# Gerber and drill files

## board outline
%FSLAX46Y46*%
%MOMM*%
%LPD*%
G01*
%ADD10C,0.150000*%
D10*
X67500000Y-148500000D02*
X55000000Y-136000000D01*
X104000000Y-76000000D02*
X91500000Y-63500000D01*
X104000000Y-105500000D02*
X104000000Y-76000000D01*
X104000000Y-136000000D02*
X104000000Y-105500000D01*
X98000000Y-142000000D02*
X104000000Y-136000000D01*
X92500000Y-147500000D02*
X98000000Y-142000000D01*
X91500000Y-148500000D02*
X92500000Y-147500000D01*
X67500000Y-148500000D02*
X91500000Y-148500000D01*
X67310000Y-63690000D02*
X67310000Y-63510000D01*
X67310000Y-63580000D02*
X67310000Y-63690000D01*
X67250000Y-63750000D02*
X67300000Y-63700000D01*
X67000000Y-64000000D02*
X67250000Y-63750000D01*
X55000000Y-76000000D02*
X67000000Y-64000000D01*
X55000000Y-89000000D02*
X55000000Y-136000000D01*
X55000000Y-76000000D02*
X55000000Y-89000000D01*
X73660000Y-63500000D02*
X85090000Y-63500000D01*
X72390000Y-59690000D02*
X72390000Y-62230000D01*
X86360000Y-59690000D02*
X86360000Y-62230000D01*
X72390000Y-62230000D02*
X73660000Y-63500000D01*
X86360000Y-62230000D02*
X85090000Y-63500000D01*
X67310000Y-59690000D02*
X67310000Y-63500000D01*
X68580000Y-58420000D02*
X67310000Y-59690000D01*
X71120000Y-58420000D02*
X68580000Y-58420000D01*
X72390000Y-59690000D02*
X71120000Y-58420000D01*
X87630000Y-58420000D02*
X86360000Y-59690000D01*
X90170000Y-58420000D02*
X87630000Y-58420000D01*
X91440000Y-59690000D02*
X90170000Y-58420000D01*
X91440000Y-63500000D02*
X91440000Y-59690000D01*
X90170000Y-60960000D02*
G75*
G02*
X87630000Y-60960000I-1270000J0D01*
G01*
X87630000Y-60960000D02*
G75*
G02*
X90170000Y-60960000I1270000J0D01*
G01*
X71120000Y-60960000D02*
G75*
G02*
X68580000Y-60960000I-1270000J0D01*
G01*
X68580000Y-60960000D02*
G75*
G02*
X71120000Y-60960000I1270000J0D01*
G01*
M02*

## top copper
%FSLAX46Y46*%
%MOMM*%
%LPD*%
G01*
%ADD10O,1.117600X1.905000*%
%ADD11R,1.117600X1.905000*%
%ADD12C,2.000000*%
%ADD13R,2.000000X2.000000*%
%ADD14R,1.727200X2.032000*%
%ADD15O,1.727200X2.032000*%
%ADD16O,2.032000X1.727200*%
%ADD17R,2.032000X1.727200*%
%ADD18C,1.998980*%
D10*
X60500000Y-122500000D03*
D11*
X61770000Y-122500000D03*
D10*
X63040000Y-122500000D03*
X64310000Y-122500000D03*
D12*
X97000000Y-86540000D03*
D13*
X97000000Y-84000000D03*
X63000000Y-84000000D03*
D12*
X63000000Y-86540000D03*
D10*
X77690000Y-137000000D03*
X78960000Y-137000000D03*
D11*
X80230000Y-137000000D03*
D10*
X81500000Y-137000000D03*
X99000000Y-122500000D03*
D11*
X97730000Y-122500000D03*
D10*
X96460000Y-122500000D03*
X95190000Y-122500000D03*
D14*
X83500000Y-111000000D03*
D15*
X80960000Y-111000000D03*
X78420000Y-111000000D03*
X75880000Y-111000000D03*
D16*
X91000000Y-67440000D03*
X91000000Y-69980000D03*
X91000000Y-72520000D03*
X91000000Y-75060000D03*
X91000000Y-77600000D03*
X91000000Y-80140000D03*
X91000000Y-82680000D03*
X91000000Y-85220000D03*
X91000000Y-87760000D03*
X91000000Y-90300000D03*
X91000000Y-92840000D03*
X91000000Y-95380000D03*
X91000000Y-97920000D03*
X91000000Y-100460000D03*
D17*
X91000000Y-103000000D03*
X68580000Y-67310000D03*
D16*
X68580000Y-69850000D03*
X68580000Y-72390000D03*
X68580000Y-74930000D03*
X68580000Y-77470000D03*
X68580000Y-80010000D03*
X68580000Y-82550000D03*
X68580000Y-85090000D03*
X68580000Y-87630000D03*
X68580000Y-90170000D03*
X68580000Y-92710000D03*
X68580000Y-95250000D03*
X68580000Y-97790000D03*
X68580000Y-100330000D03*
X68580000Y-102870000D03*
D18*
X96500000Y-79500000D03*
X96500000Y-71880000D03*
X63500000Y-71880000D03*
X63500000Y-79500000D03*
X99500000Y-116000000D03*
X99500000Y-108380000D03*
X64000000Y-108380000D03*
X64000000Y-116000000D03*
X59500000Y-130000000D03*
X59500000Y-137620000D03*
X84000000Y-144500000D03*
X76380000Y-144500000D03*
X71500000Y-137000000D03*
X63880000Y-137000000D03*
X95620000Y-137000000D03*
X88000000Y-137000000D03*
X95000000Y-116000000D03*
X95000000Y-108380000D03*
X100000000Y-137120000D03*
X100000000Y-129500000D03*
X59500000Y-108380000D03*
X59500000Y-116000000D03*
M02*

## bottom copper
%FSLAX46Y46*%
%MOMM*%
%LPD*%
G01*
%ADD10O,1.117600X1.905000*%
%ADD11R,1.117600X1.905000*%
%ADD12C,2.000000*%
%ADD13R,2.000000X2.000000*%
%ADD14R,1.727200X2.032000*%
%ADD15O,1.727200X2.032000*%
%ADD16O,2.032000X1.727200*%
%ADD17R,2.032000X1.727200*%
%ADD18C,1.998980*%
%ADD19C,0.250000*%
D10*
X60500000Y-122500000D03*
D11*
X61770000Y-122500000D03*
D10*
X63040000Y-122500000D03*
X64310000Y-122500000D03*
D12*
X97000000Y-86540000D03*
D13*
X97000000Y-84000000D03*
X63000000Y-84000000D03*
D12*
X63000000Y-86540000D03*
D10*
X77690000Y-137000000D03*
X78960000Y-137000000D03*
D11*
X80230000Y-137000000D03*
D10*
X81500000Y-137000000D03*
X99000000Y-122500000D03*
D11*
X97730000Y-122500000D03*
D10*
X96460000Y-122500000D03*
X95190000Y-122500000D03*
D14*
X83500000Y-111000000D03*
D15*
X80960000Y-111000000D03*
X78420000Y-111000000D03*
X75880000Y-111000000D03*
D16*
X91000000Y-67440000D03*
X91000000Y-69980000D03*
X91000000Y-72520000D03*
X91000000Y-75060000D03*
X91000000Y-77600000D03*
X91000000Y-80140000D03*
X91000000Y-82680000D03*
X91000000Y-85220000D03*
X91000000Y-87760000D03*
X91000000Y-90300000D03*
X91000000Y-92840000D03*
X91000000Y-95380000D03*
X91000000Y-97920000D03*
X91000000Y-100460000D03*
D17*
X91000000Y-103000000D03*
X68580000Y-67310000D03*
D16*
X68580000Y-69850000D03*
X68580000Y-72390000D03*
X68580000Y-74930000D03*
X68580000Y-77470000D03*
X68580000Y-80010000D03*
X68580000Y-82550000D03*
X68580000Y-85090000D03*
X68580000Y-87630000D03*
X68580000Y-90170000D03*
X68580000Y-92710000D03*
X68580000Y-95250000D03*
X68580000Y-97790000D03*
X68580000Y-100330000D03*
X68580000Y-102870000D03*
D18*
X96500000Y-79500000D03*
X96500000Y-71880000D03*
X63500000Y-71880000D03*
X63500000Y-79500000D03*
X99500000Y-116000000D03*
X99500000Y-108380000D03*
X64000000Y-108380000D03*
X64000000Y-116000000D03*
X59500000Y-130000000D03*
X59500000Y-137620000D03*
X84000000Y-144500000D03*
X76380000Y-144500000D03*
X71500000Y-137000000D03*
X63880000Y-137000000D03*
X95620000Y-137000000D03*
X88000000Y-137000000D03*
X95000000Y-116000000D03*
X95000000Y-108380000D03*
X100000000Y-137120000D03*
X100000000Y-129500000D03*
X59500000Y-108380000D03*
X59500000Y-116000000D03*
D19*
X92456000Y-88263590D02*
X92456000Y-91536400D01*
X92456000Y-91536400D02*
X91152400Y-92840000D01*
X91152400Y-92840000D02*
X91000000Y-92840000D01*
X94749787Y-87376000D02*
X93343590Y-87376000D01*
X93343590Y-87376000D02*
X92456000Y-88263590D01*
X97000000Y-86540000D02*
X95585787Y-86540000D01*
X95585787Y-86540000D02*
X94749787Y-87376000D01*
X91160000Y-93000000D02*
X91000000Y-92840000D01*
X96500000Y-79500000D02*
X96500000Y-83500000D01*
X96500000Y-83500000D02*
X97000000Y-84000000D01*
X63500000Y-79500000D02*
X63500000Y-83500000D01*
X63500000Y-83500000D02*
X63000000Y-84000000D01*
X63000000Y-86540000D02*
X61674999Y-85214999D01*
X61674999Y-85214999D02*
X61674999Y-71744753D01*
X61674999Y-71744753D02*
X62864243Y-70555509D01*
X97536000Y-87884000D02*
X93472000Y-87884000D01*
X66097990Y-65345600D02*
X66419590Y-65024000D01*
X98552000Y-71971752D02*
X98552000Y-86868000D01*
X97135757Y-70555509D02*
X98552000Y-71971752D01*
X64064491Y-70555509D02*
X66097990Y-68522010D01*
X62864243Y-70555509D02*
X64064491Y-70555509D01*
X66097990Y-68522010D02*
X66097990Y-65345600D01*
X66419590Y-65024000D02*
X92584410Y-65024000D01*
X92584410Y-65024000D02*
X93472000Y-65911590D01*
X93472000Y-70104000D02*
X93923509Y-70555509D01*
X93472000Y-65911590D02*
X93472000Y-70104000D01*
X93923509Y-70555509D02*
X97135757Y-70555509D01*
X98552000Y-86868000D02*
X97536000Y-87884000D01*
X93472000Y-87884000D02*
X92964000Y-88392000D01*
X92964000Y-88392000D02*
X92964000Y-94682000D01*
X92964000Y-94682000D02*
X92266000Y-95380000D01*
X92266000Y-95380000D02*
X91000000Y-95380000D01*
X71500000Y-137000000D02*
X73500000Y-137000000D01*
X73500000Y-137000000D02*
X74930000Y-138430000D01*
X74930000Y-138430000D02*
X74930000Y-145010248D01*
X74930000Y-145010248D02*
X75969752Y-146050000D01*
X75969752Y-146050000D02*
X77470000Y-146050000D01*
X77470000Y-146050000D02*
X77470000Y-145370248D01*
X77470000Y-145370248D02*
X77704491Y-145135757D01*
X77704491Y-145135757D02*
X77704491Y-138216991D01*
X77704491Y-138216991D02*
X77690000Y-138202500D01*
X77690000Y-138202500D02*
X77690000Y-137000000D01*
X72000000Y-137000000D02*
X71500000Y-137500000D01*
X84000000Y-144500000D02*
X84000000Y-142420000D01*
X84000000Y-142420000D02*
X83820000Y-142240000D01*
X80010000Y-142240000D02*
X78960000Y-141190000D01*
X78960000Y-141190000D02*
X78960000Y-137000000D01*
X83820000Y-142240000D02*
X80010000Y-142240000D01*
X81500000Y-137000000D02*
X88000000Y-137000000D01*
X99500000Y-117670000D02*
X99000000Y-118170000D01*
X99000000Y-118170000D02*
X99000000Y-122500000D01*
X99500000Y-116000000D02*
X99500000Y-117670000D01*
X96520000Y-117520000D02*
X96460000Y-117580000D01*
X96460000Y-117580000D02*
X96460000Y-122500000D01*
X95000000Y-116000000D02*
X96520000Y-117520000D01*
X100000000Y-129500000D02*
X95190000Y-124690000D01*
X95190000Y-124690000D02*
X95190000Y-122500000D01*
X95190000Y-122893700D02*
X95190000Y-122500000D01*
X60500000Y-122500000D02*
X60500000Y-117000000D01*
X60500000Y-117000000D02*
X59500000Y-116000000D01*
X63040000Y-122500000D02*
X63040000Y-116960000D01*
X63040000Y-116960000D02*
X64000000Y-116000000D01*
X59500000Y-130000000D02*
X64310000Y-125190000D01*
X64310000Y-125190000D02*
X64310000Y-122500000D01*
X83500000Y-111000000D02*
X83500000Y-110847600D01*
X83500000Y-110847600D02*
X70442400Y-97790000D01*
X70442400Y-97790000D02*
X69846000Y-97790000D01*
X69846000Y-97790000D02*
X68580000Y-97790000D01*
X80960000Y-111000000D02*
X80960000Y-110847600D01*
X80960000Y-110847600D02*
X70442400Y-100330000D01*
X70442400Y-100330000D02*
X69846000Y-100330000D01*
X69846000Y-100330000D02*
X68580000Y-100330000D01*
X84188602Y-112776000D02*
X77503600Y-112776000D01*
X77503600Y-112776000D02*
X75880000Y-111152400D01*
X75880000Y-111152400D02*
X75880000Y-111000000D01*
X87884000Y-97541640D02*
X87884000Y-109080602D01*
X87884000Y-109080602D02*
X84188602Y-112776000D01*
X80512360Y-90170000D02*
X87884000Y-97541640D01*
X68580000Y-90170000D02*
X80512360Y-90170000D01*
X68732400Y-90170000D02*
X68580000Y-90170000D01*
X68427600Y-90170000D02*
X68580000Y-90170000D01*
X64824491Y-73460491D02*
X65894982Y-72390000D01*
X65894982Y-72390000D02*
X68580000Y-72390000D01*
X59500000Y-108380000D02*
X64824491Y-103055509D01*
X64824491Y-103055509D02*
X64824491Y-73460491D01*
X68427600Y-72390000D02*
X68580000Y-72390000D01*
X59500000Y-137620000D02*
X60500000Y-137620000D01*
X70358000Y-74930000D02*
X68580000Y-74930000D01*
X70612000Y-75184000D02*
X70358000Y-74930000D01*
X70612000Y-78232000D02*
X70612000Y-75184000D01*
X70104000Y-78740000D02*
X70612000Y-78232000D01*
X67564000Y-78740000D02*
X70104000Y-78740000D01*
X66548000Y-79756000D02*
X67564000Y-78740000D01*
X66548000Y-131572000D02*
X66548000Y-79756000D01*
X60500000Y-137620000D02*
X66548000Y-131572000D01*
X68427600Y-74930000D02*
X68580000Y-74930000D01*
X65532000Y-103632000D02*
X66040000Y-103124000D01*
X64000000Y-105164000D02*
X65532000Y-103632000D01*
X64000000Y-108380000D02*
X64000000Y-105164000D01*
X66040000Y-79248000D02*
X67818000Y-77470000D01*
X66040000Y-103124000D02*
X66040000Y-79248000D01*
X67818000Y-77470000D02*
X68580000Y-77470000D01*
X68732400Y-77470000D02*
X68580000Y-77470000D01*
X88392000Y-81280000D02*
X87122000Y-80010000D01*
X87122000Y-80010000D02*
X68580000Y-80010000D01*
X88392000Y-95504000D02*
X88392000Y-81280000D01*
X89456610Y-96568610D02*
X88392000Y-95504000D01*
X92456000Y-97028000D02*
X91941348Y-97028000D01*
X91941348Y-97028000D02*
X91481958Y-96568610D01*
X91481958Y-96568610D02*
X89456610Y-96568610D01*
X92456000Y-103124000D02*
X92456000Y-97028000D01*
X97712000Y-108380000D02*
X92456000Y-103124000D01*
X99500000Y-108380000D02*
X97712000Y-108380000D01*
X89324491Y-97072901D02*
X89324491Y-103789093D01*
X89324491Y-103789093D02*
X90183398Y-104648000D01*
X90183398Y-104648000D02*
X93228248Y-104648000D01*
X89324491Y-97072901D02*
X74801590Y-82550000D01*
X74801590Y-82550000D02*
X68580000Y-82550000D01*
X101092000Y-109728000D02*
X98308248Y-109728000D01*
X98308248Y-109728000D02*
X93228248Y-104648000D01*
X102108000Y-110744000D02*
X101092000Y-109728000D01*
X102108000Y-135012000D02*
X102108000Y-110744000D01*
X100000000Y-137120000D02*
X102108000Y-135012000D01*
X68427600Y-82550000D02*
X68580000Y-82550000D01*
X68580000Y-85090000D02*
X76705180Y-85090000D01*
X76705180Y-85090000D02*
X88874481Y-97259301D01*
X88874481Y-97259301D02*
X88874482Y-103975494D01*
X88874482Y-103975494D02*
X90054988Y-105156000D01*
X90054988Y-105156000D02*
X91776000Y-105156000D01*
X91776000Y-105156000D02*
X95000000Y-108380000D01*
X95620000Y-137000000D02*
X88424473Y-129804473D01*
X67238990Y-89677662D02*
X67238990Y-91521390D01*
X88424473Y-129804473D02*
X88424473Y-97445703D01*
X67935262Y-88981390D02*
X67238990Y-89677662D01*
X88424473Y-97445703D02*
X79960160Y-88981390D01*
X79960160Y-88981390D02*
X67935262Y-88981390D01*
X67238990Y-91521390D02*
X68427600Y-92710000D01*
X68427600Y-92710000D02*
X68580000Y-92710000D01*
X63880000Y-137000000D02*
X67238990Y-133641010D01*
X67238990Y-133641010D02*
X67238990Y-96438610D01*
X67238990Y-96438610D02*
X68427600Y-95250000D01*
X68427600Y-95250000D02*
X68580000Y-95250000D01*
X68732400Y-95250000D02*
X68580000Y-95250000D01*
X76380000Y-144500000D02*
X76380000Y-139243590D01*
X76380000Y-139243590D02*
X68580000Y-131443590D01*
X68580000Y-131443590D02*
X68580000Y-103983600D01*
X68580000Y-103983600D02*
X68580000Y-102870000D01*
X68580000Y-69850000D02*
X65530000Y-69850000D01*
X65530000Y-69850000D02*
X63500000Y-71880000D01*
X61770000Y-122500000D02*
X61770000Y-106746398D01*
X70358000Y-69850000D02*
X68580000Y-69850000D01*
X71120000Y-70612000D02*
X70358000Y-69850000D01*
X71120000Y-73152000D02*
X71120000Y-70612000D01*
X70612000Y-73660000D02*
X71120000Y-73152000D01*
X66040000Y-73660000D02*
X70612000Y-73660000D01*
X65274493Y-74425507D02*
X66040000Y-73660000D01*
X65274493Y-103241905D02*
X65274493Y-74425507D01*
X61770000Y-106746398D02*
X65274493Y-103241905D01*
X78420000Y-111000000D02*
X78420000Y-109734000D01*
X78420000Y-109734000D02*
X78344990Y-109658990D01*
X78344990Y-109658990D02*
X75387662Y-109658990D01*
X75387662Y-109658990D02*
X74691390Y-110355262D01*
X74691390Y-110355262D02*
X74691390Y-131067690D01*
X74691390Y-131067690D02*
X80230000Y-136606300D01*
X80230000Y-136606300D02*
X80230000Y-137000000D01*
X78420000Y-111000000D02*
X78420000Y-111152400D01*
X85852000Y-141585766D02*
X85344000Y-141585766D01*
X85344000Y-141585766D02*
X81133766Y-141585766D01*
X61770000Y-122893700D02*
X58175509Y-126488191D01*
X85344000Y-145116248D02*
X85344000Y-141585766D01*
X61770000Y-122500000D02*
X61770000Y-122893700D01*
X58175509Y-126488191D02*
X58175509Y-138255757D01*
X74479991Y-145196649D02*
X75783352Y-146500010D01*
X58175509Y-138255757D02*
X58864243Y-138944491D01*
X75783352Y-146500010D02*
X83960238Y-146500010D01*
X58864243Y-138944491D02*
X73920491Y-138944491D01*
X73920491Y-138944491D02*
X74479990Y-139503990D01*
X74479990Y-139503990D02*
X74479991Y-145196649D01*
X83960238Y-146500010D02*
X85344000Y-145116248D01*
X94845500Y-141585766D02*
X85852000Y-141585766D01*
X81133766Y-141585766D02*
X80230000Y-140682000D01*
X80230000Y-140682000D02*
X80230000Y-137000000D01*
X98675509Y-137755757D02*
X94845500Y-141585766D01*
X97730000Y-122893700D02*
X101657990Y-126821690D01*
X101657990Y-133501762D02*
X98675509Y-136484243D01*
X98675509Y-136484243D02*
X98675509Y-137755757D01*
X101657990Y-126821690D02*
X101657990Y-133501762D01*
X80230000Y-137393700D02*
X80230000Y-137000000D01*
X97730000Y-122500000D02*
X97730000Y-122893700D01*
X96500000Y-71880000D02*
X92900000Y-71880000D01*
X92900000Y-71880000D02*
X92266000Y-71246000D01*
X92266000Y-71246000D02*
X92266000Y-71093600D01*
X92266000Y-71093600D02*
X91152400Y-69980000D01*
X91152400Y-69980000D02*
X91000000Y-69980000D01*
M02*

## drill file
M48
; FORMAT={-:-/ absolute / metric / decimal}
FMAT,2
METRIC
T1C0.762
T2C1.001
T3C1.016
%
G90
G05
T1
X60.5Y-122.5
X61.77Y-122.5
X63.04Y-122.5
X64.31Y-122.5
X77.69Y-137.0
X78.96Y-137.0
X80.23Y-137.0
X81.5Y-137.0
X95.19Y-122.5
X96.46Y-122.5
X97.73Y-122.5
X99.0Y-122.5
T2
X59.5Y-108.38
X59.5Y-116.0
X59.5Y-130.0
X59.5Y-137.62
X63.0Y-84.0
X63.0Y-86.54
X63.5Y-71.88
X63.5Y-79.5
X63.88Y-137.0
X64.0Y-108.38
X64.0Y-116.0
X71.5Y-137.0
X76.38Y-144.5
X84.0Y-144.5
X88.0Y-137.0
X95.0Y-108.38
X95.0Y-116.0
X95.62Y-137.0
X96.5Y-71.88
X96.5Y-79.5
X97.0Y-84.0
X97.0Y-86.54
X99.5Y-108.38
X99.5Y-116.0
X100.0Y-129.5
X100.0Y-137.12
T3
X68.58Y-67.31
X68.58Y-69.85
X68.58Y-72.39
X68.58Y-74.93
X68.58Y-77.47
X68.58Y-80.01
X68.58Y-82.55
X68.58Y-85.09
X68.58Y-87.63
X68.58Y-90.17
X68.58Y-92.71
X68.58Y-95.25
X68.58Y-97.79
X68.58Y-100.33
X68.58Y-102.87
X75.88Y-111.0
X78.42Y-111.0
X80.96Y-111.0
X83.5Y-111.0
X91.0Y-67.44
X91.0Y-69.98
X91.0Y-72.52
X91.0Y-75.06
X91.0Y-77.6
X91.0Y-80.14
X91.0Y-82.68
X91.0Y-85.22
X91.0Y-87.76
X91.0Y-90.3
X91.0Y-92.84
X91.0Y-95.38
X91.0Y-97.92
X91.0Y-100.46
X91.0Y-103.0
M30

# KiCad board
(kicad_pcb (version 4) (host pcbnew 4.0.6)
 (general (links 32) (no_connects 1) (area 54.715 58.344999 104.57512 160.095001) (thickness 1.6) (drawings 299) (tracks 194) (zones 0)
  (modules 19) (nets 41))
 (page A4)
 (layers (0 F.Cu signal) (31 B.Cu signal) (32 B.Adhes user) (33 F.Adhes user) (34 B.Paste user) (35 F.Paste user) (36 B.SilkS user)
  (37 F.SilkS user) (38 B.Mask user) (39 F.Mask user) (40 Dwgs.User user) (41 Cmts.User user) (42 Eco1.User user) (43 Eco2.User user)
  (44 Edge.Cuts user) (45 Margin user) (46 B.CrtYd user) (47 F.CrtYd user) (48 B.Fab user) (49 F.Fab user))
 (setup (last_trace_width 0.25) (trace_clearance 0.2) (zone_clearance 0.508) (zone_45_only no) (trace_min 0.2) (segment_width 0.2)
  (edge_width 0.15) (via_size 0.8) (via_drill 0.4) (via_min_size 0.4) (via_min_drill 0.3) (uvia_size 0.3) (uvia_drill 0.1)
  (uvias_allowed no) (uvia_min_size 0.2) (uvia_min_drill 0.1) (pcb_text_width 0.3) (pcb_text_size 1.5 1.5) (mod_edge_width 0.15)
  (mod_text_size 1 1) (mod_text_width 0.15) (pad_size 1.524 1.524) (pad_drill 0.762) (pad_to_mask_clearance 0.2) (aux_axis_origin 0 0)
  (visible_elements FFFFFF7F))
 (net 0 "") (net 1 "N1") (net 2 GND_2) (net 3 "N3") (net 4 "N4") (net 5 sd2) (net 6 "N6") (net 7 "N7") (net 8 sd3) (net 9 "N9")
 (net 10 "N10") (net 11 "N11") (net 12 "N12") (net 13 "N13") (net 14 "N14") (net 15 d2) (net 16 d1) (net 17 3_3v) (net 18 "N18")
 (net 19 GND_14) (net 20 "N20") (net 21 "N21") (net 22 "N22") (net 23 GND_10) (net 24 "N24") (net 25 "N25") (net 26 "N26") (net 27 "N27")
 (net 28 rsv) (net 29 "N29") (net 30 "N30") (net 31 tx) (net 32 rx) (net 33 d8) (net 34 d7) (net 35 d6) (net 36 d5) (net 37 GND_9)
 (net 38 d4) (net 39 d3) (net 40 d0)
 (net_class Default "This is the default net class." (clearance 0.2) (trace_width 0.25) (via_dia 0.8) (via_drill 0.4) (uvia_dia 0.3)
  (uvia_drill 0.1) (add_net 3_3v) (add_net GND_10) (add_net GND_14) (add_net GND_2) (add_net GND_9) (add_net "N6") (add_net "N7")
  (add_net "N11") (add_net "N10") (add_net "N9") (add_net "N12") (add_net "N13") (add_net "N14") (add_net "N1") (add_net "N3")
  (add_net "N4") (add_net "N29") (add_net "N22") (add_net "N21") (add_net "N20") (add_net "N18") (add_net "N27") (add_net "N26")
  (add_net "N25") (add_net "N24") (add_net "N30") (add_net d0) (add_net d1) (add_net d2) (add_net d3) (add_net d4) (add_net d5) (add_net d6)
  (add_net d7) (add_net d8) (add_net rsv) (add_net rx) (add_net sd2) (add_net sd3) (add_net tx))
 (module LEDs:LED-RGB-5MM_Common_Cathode (layer F.Cu) (at 60.5 122.5 90)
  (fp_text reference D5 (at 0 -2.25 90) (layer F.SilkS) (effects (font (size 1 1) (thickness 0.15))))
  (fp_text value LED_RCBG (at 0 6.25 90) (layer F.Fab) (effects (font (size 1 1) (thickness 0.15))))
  (pad 1 thru_hole oval (at 0 0 90) (size 1.905 1.1176) (drill 0.762) (layers *.Cu *.Mask F.SilkS) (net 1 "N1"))
  (pad 2 thru_hole rect (at 0 1.27 90) (size 1.905 1.1176) (drill 0.762) (layers *.Cu *.Mask F.SilkS) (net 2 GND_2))
  (pad 3 thru_hole oval (at 0 2.54 90) (size 1.905 1.1176) (drill 0.762) (layers *.Cu *.Mask F.SilkS) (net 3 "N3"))
  (pad 4 thru_hole oval (at 0 3.81 90) (size 1.905 1.1176) (drill 0.762) (layers *.Cu *.Mask F.SilkS) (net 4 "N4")))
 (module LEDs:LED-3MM (layer F.Cu) (at 97 84 270)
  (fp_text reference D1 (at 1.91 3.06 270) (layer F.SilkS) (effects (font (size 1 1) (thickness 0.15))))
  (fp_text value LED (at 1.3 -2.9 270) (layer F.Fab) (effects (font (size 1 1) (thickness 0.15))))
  (pad 2 thru_hole circle (at 2.54 0 270) (size 2 2) (drill 1.00076) (layers *.Cu *.Mask F.SilkS) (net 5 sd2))
  (pad 1 thru_hole rect (at 0 0) (size 2 2) (drill 1.00076) (layers *.Cu *.Mask F.SilkS) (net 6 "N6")))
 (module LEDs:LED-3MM (layer F.Cu) (at 63 84 270)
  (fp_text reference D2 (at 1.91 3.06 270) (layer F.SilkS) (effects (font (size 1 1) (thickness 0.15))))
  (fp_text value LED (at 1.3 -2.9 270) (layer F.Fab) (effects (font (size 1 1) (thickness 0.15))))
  (pad 1 thru_hole rect (at 0 0) (size 2 2) (drill 1.00076) (layers *.Cu *.Mask F.SilkS) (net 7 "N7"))
  (pad 2 thru_hole circle (at 2.54 0 270) (size 2 2) (drill 1.00076) (layers *.Cu *.Mask F.SilkS) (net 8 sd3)))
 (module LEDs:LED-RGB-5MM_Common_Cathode (layer F.Cu) (at 81.5 137 270)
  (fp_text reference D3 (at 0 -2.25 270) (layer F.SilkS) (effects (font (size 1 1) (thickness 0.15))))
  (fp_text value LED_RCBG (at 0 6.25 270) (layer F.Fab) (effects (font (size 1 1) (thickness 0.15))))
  (pad 4 thru_hole oval (at 0 3.81 270) (size 1.905 1.1176) (drill 0.762) (layers *.Cu *.Mask F.SilkS) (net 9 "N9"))
  (pad 3 thru_hole oval (at 0 2.54 270) (size 1.905 1.1176) (drill 0.762) (layers *.Cu *.Mask F.SilkS) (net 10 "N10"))
  (pad 2 thru_hole rect (at 0 1.27 270) (size 1.905 1.1176) (drill 0.762) (layers *.Cu *.Mask F.SilkS) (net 2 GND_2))
  (pad 1 thru_hole oval (at 0 0 270) (size 1.905 1.1176) (drill 0.762) (layers *.Cu *.Mask F.SilkS) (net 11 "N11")))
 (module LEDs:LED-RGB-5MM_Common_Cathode (layer F.Cu) (at 99 122.5 270)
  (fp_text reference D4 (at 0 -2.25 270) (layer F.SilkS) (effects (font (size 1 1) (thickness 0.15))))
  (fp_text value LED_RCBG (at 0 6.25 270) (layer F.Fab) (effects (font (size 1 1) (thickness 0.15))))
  (pad 1 thru_hole oval (at 0 0 270) (size 1.905 1.1176) (drill 0.762) (layers *.Cu *.Mask F.SilkS) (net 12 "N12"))
  (pad 2 thru_hole rect (at 0 1.27 270) (size 1.905 1.1176) (drill 0.762) (layers *.Cu *.Mask F.SilkS) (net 2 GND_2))
  (pad 3 thru_hole oval (at 0 2.54 270) (size 1.905 1.1176) (drill 0.762) (layers *.Cu *.Mask F.SilkS) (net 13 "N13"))
  (pad 4 thru_hole oval (at 0 3.81 270) (size 1.905 1.1176) (drill 0.762) (layers *.Cu *.Mask F.SilkS) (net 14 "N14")))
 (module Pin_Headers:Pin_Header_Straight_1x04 (layer F.Cu) (at 83.5 111 270)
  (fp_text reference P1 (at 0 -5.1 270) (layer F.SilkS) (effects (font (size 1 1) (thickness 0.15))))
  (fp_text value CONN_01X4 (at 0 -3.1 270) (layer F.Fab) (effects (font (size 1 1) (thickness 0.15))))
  (pad 1 thru_hole rect (at 0 0 270) (size 2.032 1.7272) (drill 1.016) (layers *.Cu *.Mask F.SilkS) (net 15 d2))
  (pad 2 thru_hole oval (at 0 2.54 270) (size 2.032 1.7272) (drill 1.016) (layers *.Cu *.Mask F.SilkS) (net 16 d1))
  (pad 3 thru_hole oval (at 0 5.08 270) (size 2.032 1.7272) (drill 1.016) (layers *.Cu *.Mask F.SilkS) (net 2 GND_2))
  (pad 4 thru_hole oval (at 0 7.62 270) (size 2.032 1.7272) (drill 1.016) (layers *.Cu *.Mask F.SilkS) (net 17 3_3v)))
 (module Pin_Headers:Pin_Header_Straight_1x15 (layer F.Cu) (at 91 103 180)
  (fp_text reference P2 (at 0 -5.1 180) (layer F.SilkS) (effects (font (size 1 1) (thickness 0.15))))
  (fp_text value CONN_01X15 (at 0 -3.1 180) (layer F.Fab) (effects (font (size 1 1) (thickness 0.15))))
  (pad 15 thru_hole oval (at 0 35.56 180) (size 2.032 1.7272) (drill 1.016) (layers *.Cu *.Mask F.SilkS) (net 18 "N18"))
  (pad 14 thru_hole oval (at 0 33.02 180) (size 2.032 1.7272) (drill 1.016) (layers *.Cu *.Mask F.SilkS) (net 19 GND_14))
  (pad 13 thru_hole oval (at 0 30.48 180) (size 2.032 1.7272) (drill 1.016) (layers *.Cu *.Mask F.SilkS) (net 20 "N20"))
  (pad 12 thru_hole oval (at 0 27.94 180) (size 2.032 1.7272) (drill 1.016) (layers *.Cu *.Mask F.SilkS) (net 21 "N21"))
  (pad 11 thru_hole oval (at 0 25.4 180) (size 2.032 1.7272) (drill 1.016) (layers *.Cu *.Mask F.SilkS) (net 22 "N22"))
  (pad 10 thru_hole oval (at 0 22.86 180) (size 2.032 1.7272) (drill 1.016) (layers *.Cu *.Mask F.SilkS) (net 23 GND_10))
  (pad 9 thru_hole oval (at 0 20.32 180) (size 2.032 1.7272) (drill 1.016) (layers *.Cu *.Mask F.SilkS) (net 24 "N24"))
  (pad 8 thru_hole oval (at 0 17.78 180) (size 2.032 1.7272) (drill 1.016) (layers *.Cu *.Mask F.SilkS) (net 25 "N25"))
  (pad 7 thru_hole oval (at 0 15.24 180) (size 2.032 1.7272) (drill 1.016) (layers *.Cu *.Mask F.SilkS) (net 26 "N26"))
  (pad 6 thru_hole oval (at 0 12.7 180) (size 2.032 1.7272) (drill 1.016) (layers *.Cu *.Mask F.SilkS) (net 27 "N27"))
  (pad 5 thru_hole oval (at 0 10.16 180) (size 2.032 1.7272) (drill 1.016) (layers *.Cu *.Mask F.SilkS) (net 5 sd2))
  (pad 4 thru_hole oval (at 0 7.62 180) (size 2.032 1.7272) (drill 1.016) (layers *.Cu *.Mask F.SilkS) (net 8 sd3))
  (pad 3 thru_hole oval (at 0 5.08 180) (size 2.032 1.7272) (drill 1.016) (layers *.Cu *.Mask F.SilkS) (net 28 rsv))
  (pad 2 thru_hole oval (at 0 2.54 180) (size 2.032 1.7272) (drill 1.016) (layers *.Cu *.Mask F.SilkS) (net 28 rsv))
  (pad 1 thru_hole rect (at 0 0 180) (size 2.032 1.7272) (drill 1.016) (layers *.Cu *.Mask F.SilkS) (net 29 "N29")))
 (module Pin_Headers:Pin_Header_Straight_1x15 (layer F.Cu) (at 68.58 67.31)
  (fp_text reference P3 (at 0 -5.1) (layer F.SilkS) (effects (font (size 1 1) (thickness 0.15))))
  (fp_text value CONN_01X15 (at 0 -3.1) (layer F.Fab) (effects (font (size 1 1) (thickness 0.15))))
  (pad 1 thru_hole rect (at 0 0) (size 2.032 1.7272) (drill 1.016) (layers *.Cu *.Mask F.SilkS) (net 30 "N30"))
  (pad 2 thru_hole oval (at 0 2.54) (size 2.032 1.7272) (drill 1.016) (layers *.Cu *.Mask F.SilkS) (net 2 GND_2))
  (pad 3 thru_hole oval (at 0 5.08) (size 2.032 1.7272) (drill 1.016) (layers *.Cu *.Mask F.SilkS) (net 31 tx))
  (pad 4 thru_hole oval (at 0 7.62) (size 2.032 1.7272) (drill 1.016) (layers *.Cu *.Mask F.SilkS) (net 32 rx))
  (pad 5 thru_hole oval (at 0 10.16) (size 2.032 1.7272) (drill 1.016) (layers *.Cu *.Mask F.SilkS) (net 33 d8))
  (pad 6 thru_hole oval (at 0 12.7) (size 2.032 1.7272) (drill 1.016) (layers *.Cu *.Mask F.SilkS) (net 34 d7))
  (pad 7 thru_hole oval (at 0 15.24) (size 2.032 1.7272) (drill 1.016) (layers *.Cu *.Mask F.SilkS) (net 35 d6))
  (pad 8 thru_hole oval (at 0 17.78) (size 2.032 1.7272) (drill 1.016) (layers *.Cu *.Mask F.SilkS) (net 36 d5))
  (pad 9 thru_hole oval (at 0 20.32) (size 2.032 1.7272) (drill 1.016) (layers *.Cu *.Mask F.SilkS) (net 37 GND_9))
  (pad 10 thru_hole oval (at 0 22.86) (size 2.032 1.7272) (drill 1.016) (layers *.Cu *.Mask F.SilkS) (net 17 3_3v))
  (pad 11 thru_hole oval (at 0 25.4) (size 2.032 1.7272) (drill 1.016) (layers *.Cu *.Mask F.SilkS) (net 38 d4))
  (pad 12 thru_hole oval (at 0 27.94) (size 2.032 1.7272) (drill 1.016) (layers *.Cu *.Mask F.SilkS) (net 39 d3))
  (pad 13 thru_hole oval (at 0 30.48) (size 2.032 1.7272) (drill 1.016) (layers *.Cu *.Mask F.SilkS) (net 15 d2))
  (pad 14 thru_hole oval (at 0 33.02) (size 2.032 1.7272) (drill 1.016) (layers *.Cu *.Mask F.SilkS) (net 16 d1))
  (pad 15 thru_hole oval (at 0 35.56) (size 2.032 1.7272) (drill 1.016) (layers *.Cu *.Mask F.SilkS) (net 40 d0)))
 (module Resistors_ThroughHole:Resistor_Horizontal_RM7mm (layer F.Cu) (at 96.5 79.5 90)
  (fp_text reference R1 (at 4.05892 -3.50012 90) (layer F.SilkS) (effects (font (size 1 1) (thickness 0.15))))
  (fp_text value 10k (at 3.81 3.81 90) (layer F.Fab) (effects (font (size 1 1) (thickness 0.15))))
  (pad 1 thru_hole circle (at 0 0 90) (size 1.99898 1.99898) (drill 1.00076) (layers *.Cu *.SilkS *.Mask) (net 6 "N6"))
  (pad 2 thru_hole circle (at 7.62 0 90) (size 1.99898 1.99898) (drill 1.00076) (layers *.Cu *.SilkS *.Mask) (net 19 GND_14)))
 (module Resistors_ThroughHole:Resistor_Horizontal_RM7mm (layer F.Cu) (at 63.5 79.5 90)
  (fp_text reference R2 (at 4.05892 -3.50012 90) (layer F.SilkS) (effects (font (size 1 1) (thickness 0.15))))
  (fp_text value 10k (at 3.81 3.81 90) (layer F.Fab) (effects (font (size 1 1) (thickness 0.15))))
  (pad 2 thru_hole circle (at 7.62 0 90) (size 1.99898 1.99898) (drill 1.00076) (layers *.Cu *.SilkS *.Mask) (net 2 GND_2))
  (pad 1 thru_hole circle (at 0 0 90) (size 1.99898 1.99898) (drill 1.00076) (layers *.Cu *.SilkS *.Mask) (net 7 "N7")))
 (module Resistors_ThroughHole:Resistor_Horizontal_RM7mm (layer F.Cu) (at 99.5 116 90)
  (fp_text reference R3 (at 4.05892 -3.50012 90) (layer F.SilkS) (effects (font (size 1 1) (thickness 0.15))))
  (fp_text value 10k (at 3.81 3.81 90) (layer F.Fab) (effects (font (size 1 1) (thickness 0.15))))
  (pad 1 thru_hole circle (at 0 0 90) (size 1.99898 1.99898) (drill 1.00076) (layers *.Cu *.SilkS *.Mask) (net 12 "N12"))
  (pad 2 thru_hole circle (at 7.62 0 90) (size 1.99898 1.99898) (drill 1.00076) (layers *.Cu *.SilkS *.Mask) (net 34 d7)))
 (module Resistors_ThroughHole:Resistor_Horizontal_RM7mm (layer F.Cu) (at 64 116 90)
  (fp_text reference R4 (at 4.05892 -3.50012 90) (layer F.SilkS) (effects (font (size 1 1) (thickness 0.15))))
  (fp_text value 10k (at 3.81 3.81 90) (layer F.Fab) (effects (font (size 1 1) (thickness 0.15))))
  (pad 2 thru_hole circle (at 7.62 0 90) (size 1.99898 1.99898) (drill 1.00076) (layers *.Cu *.SilkS *.Mask) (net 33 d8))
  (pad 1 thru_hole circle (at 0 0 90) (size 1.99898 1.99898) (drill 1.00076) (layers *.Cu *.SilkS *.Mask) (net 3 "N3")))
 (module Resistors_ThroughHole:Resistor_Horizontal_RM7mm (layer F.Cu) (at 59.5 130 270)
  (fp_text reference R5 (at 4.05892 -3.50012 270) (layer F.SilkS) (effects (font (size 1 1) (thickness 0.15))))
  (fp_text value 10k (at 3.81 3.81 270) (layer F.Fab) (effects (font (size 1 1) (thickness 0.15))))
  (pad 1 thru_hole circle (at 0 0 270) (size 1.99898 1.99898) (drill 1.00076) (layers *.Cu *.SilkS *.Mask) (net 4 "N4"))
  (pad 2 thru_hole circle (at 7.62 0 270) (size 1.99898 1.99898) (drill 1.00076) (layers *.Cu *.SilkS *.Mask) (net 32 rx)))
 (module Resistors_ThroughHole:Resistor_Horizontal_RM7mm (layer F.Cu) (at 84 144.5 180)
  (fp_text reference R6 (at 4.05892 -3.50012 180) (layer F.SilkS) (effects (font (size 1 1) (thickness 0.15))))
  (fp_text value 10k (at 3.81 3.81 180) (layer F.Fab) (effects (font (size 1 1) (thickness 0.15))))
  (pad 1 thru_hole circle (at 0 0 180) (size 1.99898 1.99898) (drill 1.00076) (layers *.Cu *.SilkS *.Mask) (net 10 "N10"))
  (pad 2 thru_hole circle (at 7.62 0 180) (size 1.99898 1.99898) (drill 1.00076) (layers *.Cu *.SilkS *.Mask) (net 40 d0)))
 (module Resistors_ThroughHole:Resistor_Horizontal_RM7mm (layer F.Cu) (at 71.5 137 180)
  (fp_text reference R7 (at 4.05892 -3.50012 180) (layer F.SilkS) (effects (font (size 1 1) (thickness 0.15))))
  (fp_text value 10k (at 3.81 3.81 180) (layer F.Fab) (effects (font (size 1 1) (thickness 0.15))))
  (pad 1 thru_hole circle (at 0 0 180) (size 1.99898 1.99898) (drill 1.00076) (layers *.Cu *.SilkS *.Mask) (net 9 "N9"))
  (pad 2 thru_hole circle (at 7.62 0 180) (size 1.99898 1.99898) (drill 1.00076) (layers *.Cu *.SilkS *.Mask) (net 39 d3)))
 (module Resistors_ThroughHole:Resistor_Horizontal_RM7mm (layer F.Cu) (at 88 137)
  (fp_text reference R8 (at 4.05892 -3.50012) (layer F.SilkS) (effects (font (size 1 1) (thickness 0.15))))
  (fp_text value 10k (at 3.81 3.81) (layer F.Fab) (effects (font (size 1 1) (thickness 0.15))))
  (pad 2 thru_hole circle (at 7.62 0) (size 1.99898 1.99898) (drill 1.00076) (layers *.Cu *.SilkS *.Mask) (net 38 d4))
  (pad 1 thru_hole circle (at 0 0) (size 1.99898 1.99898) (drill 1.00076) (layers *.Cu *.SilkS *.Mask) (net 11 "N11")))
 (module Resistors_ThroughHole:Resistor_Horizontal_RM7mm (layer F.Cu) (at 95 116 90)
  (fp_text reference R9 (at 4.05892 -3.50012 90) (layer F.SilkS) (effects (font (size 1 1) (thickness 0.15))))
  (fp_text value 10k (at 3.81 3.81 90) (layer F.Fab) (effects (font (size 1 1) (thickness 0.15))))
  (pad 1 thru_hole circle (at 0 0 90) (size 1.99898 1.99898) (drill 1.00076) (layers *.Cu *.SilkS *.Mask) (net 13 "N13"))
  (pad 2 thru_hole circle (at 7.62 0 90) (size 1.99898 1.99898) (drill 1.00076) (layers *.Cu *.SilkS *.Mask) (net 36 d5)))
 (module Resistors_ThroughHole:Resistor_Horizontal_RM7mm (layer F.Cu) (at 100 129.5 270)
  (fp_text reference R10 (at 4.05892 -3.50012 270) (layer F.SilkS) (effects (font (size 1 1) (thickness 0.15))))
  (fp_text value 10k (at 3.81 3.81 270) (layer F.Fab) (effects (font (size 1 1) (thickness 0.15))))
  (pad 2 thru_hole circle (at 7.62 0 270) (size 1.99898 1.99898) (drill 1.00076) (layers *.Cu *.SilkS *.Mask) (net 35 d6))
  (pad 1 thru_hole circle (at 0 0 270) (size 1.99898 1.99898) (drill 1.00076) (layers *.Cu *.SilkS *.Mask) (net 14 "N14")))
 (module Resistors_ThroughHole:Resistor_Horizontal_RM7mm (layer F.Cu) (at 59.5 116 90)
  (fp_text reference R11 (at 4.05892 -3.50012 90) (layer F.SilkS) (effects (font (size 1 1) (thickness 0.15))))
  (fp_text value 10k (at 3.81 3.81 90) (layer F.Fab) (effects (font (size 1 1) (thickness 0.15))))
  (pad 2 thru_hole circle (at 7.62 0 90) (size 1.99898 1.99898) (drill 1.00076) (layers *.Cu *.SilkS *.Mask) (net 31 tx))
  (pad 1 thru_hole circle (at 0 0 90) (size 1.99898 1.99898) (drill 1.00076) (layers *.Cu *.SilkS *.Mask) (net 1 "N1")))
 (gr_line (start 67.5 148.5) (end 55 136) (angle 90) (layer Edge.Cuts) (width 0.15))
 (gr_line (start 104 76) (end 91.5 63.5) (angle 90) (layer Edge.Cuts) (width 0.15))
 (gr_line (start 104 105.5) (end 104 76) (angle 90) (layer Edge.Cuts) (width 0.15))
 (gr_line (start 104 136) (end 104 105.5) (angle 90) (layer Edge.Cuts) (width 0.15))
 (gr_line (start 98 142) (end 104 136) (angle 90) (layer Edge.Cuts) (width 0.15))
 (gr_line (start 92.5 147.5) (end 98 142) (angle 90) (layer Edge.Cuts) (width 0.15))
 (gr_line (start 91.5 148.5) (end 92.5 147.5) (angle 90) (layer Edge.Cuts) (width 0.15))
 (gr_line (start 67.5 148.5) (end 91.5 148.5) (angle 90) (layer Edge.Cuts) (width 0.15))
 (gr_line (start 67.31 63.69) (end 67.31 63.51) (angle 90) (layer Edge.Cuts) (width 0.15))
 (gr_line (start 67.31 63.58) (end 67.31 63.69) (angle 90) (layer Edge.Cuts) (width 0.15))
 (gr_line (start 67.25 63.75) (end 67.3 63.7) (angle 90) (layer Edge.Cuts) (width 0.15))
 (gr_line (start 67 64) (end 67.25 63.75) (angle 90) (layer Edge.Cuts) (width 0.15))
 (gr_line (start 55 76) (end 67 64) (angle 90) (layer Edge.Cuts) (width 0.15))
 (gr_line (start 55 89) (end 55 136) (angle 90) (layer Edge.Cuts) (width 0.15))
 (gr_line (start 55 76) (end 55 89) (angle 90) (layer Edge.Cuts) (width 0.15))
 (gr_line (start 73.66 63.5) (end 85.09 63.5) (angle 90) (layer Edge.Cuts) (width 0.15))
 (gr_line (start 72.39 59.69) (end 72.39 62.23) (angle 90) (layer Edge.Cuts) (width 0.15))
 (gr_line (start 86.36 59.69) (end 86.36 62.23) (angle 90) (layer Edge.Cuts) (width 0.15))
 (gr_line (start 72.39 62.23) (end 73.66 63.5) (angle 90) (layer Edge.Cuts) (width 0.15))
 (gr_line (start 86.36 62.23) (end 85.09 63.5) (angle 90) (layer Edge.Cuts) (width 0.15))
 (gr_line (start 67.31 59.69) (end 67.31 63.5) (angle 90) (layer Edge.Cuts) (width 0.15))
 (gr_line (start 68.58 58.42) (end 67.31 59.69) (angle 90) (layer Edge.Cuts) (width 0.15))
 (gr_line (start 71.12 58.42) (end 68.58 58.42) (angle 90) (layer Edge.Cuts) (width 0.15))
 (gr_line (start 72.39 59.69) (end 71.12 58.42) (angle 90) (layer Edge.Cuts) (width 0.15))
 (gr_line (start 87.63 58.42) (end 86.36 59.69) (angle 90) (layer Edge.Cuts) (width 0.15))
 (gr_line (start 90.17 58.42) (end 87.63 58.42) (angle 90) (layer Edge.Cuts) (width 0.15))
 (gr_line (start 91.44 59.69) (end 90.17 58.42) (angle 90) (layer Edge.Cuts) (width 0.15))
 (gr_line (start 91.44 63.5) (end 91.44 59.69) (angle 90) (layer Edge.Cuts) (width 0.15))
 (gr_circle (center 88.9 60.96) (end 88.9 62.23) (layer Edge.Cuts) (width 0.15))
 (gr_circle (center 69.85 60.96) (end 69.85 62.23) (layer Edge.Cuts) (width 0.15))
 (segment (start 92.456 88.26359) (end 92.456 91.5364) (width 0.25) (layer B.Cu) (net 5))
 (segment (start 92.456 91.5364) (end 91.1524 92.84) (width 0.25) (layer B.Cu) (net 5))
 (segment (start 91.1524 92.84) (end 91 92.84) (width 0.25) (layer B.Cu) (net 5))
 (segment (start 94.749787 87.376) (end 93.34359 87.376) (width 0.25) (layer B.Cu) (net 5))
 (segment (start 93.34359 87.376) (end 92.456 88.26359) (width 0.25) (layer B.Cu) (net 5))
 (segment (start 97 86.54) (end 95.585787 86.54) (width 0.25) (layer B.Cu) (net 5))
 (segment (start 95.585787 86.54) (end 94.749787 87.376) (width 0.25) (layer B.Cu) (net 5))
 (segment (start 91.16 93) (end 91 92.84) (width 0.25) (layer B.Cu) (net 5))
 (segment (start 96.5 79.5) (end 96.5 83.5) (width 0.25) (layer B.Cu) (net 6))
 (segment (start 96.5 83.5) (end 97 84) (width 0.25) (layer B.Cu) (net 6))
 (segment (start 63.5 79.5) (end 63.5 83.5) (width 0.25) (layer B.Cu) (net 7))
 (segment (start 63.5 83.5) (end 63 84) (width 0.25) (layer B.Cu) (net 7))
 (segment (start 63 86.54) (end 61.674999 85.214999) (width 0.25) (layer B.Cu) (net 8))
 (segment (start 61.674999 85.214999) (end 61.674999 71.744753) (width 0.25) (layer B.Cu) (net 8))
 (segment (start 61.674999 71.744753) (end 62.864243 70.555509) (width 0.25) (layer B.Cu) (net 8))
 (segment (start 97.536 87.884) (end 93.472 87.884) (width 0.25) (layer B.Cu) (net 8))
 (segment (start 66.09799 65.3456) (end 66.41959 65.024) (width 0.25) (layer B.Cu) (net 8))
 (segment (start 98.552 71.971752) (end 98.552 86.868) (width 0.25) (layer B.Cu) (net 8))
 (segment (start 97.135757 70.555509) (end 98.552 71.971752) (width 0.25) (layer B.Cu) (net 8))
 (segment (start 64.064491 70.555509) (end 66.09799 68.52201) (width 0.25) (layer B.Cu) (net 8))
 (segment (start 62.864243 70.555509) (end 64.064491 70.555509) (width 0.25) (layer B.Cu) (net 8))
 (segment (start 66.09799 68.52201) (end 66.09799 65.3456) (width 0.25) (layer B.Cu) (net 8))
 (segment (start 66.41959 65.024) (end 92.58441 65.024) (width 0.25) (layer B.Cu) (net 8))
 (segment (start 92.58441 65.024) (end 93.472 65.91159) (width 0.25) (layer B.Cu) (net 8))
 (segment (start 93.472 70.104) (end 93.923509 70.555509) (width 0.25) (layer B.Cu) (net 8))
 (segment (start 93.472 65.91159) (end 93.472 70.104) (width 0.25) (layer B.Cu) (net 8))
 (segment (start 93.923509 70.555509) (end 97.135757 70.555509) (width 0.25) (layer B.Cu) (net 8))
 (segment (start 98.552 86.868) (end 97.536 87.884) (width 0.25) (layer B.Cu) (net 8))
 (segment (start 93.472 87.884) (end 92.964 88.392) (width 0.25) (layer B.Cu) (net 8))
 (segment (start 92.964 88.392) (end 92.964 94.682) (width 0.25) (layer B.Cu) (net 8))
 (segment (start 92.964 94.682) (end 92.266 95.38) (width 0.25) (layer B.Cu) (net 8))
 (segment (start 92.266 95.38) (end 91 95.38) (width 0.25) (layer B.Cu) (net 8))
 (segment (start 71.5 137) (end 73.5 137) (width 0.25) (layer B.Cu) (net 9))
 (segment (start 73.5 137) (end 74.93 138.43) (width 0.25) (layer B.Cu) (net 9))
 (segment (start 74.93 138.43) (end 74.93 145.010248) (width 0.25) (layer B.Cu) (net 9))
 (segment (start 74.93 145.010248) (end 75.969752 146.05) (width 0.25) (layer B.Cu) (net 9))
 (segment (start 75.969752 146.05) (end 77.47 146.05) (width 0.25) (layer B.Cu) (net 9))
 (segment (start 77.47 146.05) (end 77.47 145.370248) (width 0.25) (layer B.Cu) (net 9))
 (segment (start 77.47 145.370248) (end 77.704491 145.135757) (width 0.25) (layer B.Cu) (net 9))
 (segment (start 77.704491 145.135757) (end 77.704491 138.216991) (width 0.25) (layer B.Cu) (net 9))
 (segment (start 77.704491 138.216991) (end 77.69 138.2025) (width 0.25) (layer B.Cu) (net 9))
 (segment (start 77.69 138.2025) (end 77.69 137) (width 0.25) (layer B.Cu) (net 9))
 (segment (start 72 137) (end 71.5 137.5) (width 0.25) (layer B.Cu) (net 9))
 (segment (start 84 144.5) (end 84 142.42) (width 0.25) (layer B.Cu) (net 10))
 (segment (start 84 142.42) (end 83.82 142.24) (width 0.25) (layer B.Cu) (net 10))
 (segment (start 80.01 142.24) (end 78.96 141.19) (width 0.25) (layer B.Cu) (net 10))
 (segment (start 78.96 141.19) (end 78.96 137) (width 0.25) (layer B.Cu) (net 10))
 (segment (start 83.82 142.24) (end 80.01 142.24) (width 0.25) (layer B.Cu) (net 10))
 (segment (start 81.5 137) (end 88 137) (width 0.25) (layer B.Cu) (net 11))
 (segment (start 99.5 117.67) (end 99 118.17) (width 0.25) (layer B.Cu) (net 12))
 (segment (start 99 118.17) (end 99 122.5) (width 0.25) (layer B.Cu) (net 12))
 (segment (start 99.5 116) (end 99.5 117.67) (width 0.25) (layer B.Cu) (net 12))
 (segment (start 96.52 117.52) (end 96.46 117.58) (width 0.25) (layer B.Cu) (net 13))
 (segment (start 96.46 117.58) (end 96.46 122.5) (width 0.25) (layer B.Cu) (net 13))
 (segment (start 95 116) (end 96.52 117.52) (width 0.25) (layer B.Cu) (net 13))
 (segment (start 100 129.5) (end 95.19 124.69) (width 0.25) (layer B.Cu) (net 14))
 (segment (start 95.19 124.69) (end 95.19 122.5) (width 0.25) (layer B.Cu) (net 14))
 (segment (start 95.19 122.8937) (end 95.19 122.5) (width 0.25) (layer B.Cu) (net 14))
 (segment (start 60.5 122.5) (end 60.5 117) (width 0.25) (layer B.Cu) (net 1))
 (segment (start 60.5 117) (end 59.5 116) (width 0.25) (layer B.Cu) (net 1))
 (segment (start 63.04 122.5) (end 63.04 116.96) (width 0.25) (layer B.Cu) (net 3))
 (segment (start 63.04 116.96) (end 64 116) (width 0.25) (layer B.Cu) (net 3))
 (segment (start 59.5 130) (end 64.31 125.19) (width 0.25) (layer B.Cu) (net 4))
 (segment (start 64.31 125.19) (end 64.31 122.5) (width 0.25) (layer B.Cu) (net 4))
 (segment (start 83.5 111) (end 83.5 110.8476) (width 0.25) (layer B.Cu) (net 15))
 (segment (start 83.5 110.8476) (end 70.4424 97.79) (width 0.25) (layer B.Cu) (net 15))
 (segment (start 70.4424 97.79) (end 69.846 97.79) (width 0.25) (layer B.Cu) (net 15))
 (segment (start 69.846 97.79) (end 68.58 97.79) (width 0.25) (layer B.Cu) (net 15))
 (segment (start 80.96 111) (end 80.96 110.8476) (width 0.25) (layer B.Cu) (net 16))
 (segment (start 80.96 110.8476) (end 70.4424 100.33) (width 0.25) (layer B.Cu) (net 16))
 (segment (start 70.4424 100.33) (end 69.846 100.33) (width 0.25) (layer B.Cu) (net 16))
 (segment (start 69.846 100.33) (end 68.58 100.33) (width 0.25) (layer B.Cu) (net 16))
 (segment (start 84.188602 112.776) (end 77.5036 112.776) (width 0.25) (layer B.Cu) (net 17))
 (segment (start 77.5036 112.776) (end 75.88 111.1524) (width 0.25) (layer B.Cu) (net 17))
 (segment (start 75.88 111.1524) (end 75.88 111) (width 0.25) (layer B.Cu) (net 17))
 (segment (start 87.884 97.54164) (end 87.884 109.080602) (width 0.25) (layer B.Cu) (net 17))
 (segment (start 87.884 109.080602) (end 84.188602 112.776) (width 0.25) (layer B.Cu) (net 17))
 (segment (start 80.51236 90.17) (end 87.884 97.54164) (width 0.25) (layer B.Cu) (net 17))
 (segment (start 68.58 90.17) (end 80.51236 90.17) (width 0.25) (layer B.Cu) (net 17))
 (segment (start 68.7324 90.17) (end 68.58 90.17) (width 0.25) (layer B.Cu) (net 17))
 (segment (start 68.4276 90.17) (end 68.58 90.17) (width 0.25) (layer B.Cu) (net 17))
 (segment (start 64.824491 73.460491) (end 65.894982 72.39) (width 0.25) (layer B.Cu) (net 31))
 (segment (start 65.894982 72.39) (end 68.58 72.39) (width 0.25) (layer B.Cu) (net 31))
 (segment (start 59.5 108.38) (end 64.824491 103.055509) (width 0.25) (layer B.Cu) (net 31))
 (segment (start 64.824491 103.055509) (end 64.824491 73.460491) (width 0.25) (layer B.Cu) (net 31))
 (segment (start 68.4276 72.39) (end 68.58 72.39) (width 0.25) (layer B.Cu) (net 31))
 (segment (start 59.5 137.62) (end 60.5 137.62) (width 0.25) (layer B.Cu) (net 32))
 (segment (start 70.358 74.93) (end 68.58 74.93) (width 0.25) (layer B.Cu) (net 32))
 (segment (start 70.612 75.184) (end 70.358 74.93) (width 0.25) (layer B.Cu) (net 32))
 (segment (start 70.612 78.232) (end 70.612 75.184) (width 0.25) (layer B.Cu) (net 32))
 (segment (start 70.104 78.74) (end 70.612 78.232) (width 0.25) (layer B.Cu) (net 32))
 (segment (start 67.564 78.74) (end 70.104 78.74) (width 0.25) (layer B.Cu) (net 32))
 (segment (start 66.548 79.756) (end 67.564 78.74) (width 0.25) (layer B.Cu) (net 32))
 (segment (start 66.548 131.572) (end 66.548 79.756) (width 0.25) (layer B.Cu) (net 32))
 (segment (start 60.5 137.62) (end 66.548 131.572) (width 0.25) (layer B.Cu) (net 32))
 (segment (start 68.4276 74.93) (end 68.58 74.93) (width 0.25) (layer B.Cu) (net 32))
 (segment (start 65.532 103.632) (end 66.04 103.124) (width 0.25) (layer B.Cu) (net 33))
 (segment (start 64 105.164) (end 65.532 103.632) (width 0.25) (layer B.Cu) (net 33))
 (segment (start 64 108.38) (end 64 105.164) (width 0.25) (layer B.Cu) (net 33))
 (segment (start 66.04 79.248) (end 67.818 77.47) (width 0.25) (layer B.Cu) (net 33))
 (segment (start 66.04 103.124) (end 66.04 79.248) (width 0.25) (layer B.Cu) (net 33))
 (segment (start 67.818 77.47) (end 68.58 77.47) (width 0.25) (layer B.Cu) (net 33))
 (segment (start 68.7324 77.47) (end 68.58 77.47) (width 0.25) (layer B.Cu) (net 33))
 (segment (start 88.392 81.28) (end 87.122 80.01) (width 0.25) (layer B.Cu) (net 34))
 (segment (start 87.122 80.01) (end 68.58 80.01) (width 0.25) (layer B.Cu) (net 34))
 (segment (start 88.392 95.504) (end 88.392 81.28) (width 0.25) (layer B.Cu) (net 34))
 (segment (start 89.45661 96.56861) (end 88.392 95.504) (width 0.25) (layer B.Cu) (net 34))
 (segment (start 92.456 97.028) (end 91.941348 97.028) (width 0.25) (layer B.Cu) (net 34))
 (segment (start 91.941348 97.028) (end 91.481958 96.56861) (width 0.25) (layer B.Cu) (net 34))
 (segment (start 91.481958 96.56861) (end 89.45661 96.56861) (width 0.25) (layer B.Cu) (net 34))
 (segment (start 92.456 103.124) (end 92.456 97.028) (width 0.25) (layer B.Cu) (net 34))
 (segment (start 97.712 108.38) (end 92.456 103.124) (width 0.25) (layer B.Cu) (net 34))
 (segment (start 99.5 108.38) (end 97.712 108.38) (width 0.25) (layer B.Cu) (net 34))
 (segment (start 89.324491 97.072901) (end 89.324491 103.789093) (width 0.25) (layer B.Cu) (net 35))
 (segment (start 89.324491 103.789093) (end 90.183398 104.648) (width 0.25) (layer B.Cu) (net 35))
 (segment (start 90.183398 104.648) (end 93.228248 104.648) (width 0.25) (layer B.Cu) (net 35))
 (segment (start 89.324491 97.072901) (end 74.80159 82.55) (width 0.25) (layer B.Cu) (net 35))
 (segment (start 74.80159 82.55) (end 68.58 82.55) (width 0.25) (layer B.Cu) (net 35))
 (segment (start 101.092 109.728) (end 98.308248 109.728) (width 0.25) (layer B.Cu) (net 35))
 (segment (start 98.308248 109.728) (end 93.228248 104.648) (width 0.25) (layer B.Cu) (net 35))
 (segment (start 102.108 110.744) (end 101.092 109.728) (width 0.25) (layer B.Cu) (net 35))
 (segment (start 102.108 135.012) (end 102.108 110.744) (width 0.25) (layer B.Cu) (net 35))
 (segment (start 100 137.12) (end 102.108 135.012) (width 0.25) (layer B.Cu) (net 35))
 (segment (start 68.4276 82.55) (end 68.58 82.55) (width 0.25) (layer B.Cu) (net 35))
 (segment (start 68.58 85.09) (end 76.70518 85.09) (width 0.25) (layer B.Cu) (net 36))
 (segment (start 76.70518 85.09) (end 88.874481 97.259301) (width 0.25) (layer B.Cu) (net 36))
 (segment (start 88.874481 97.259301) (end 88.874482 103.975494) (width 0.25) (layer B.Cu) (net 36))
 (segment (start 88.874482 103.975494) (end 90.054988 105.156) (width 0.25) (layer B.Cu) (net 36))
 (segment (start 90.054988 105.156) (end 91.776 105.156) (width 0.25) (layer B.Cu) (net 36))
 (segment (start 91.776 105.156) (end 95 108.38) (width 0.25) (layer B.Cu) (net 36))
 (segment (start 95.62 137) (end 88.424473 129.804473) (width 0.25) (layer B.Cu) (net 38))
 (segment (start 67.23899 89.677662) (end 67.23899 91.52139) (width 0.25) (layer B.Cu) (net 38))
 (segment (start 88.424473 129.804473) (end 88.424473 97.445703) (width 0.25) (layer B.Cu) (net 38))
 (segment (start 67.935262 88.98139) (end 67.23899 89.677662) (width 0.25) (layer B.Cu) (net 38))
 (segment (start 88.424473 97.445703) (end 79.96016 88.98139) (width 0.25) (layer B.Cu) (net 38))
 (segment (start 79.96016 88.98139) (end 67.935262 88.98139) (width 0.25) (layer B.Cu) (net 38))
 (segment (start 67.23899 91.52139) (end 68.4276 92.71) (width 0.25) (layer B.Cu) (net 38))
 (segment (start 68.4276 92.71) (end 68.58 92.71) (width 0.25) (layer B.Cu) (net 38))
 (segment (start 63.88 137) (end 67.23899 133.64101) (width 0.25) (layer B.Cu) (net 39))
 (segment (start 67.23899 133.64101) (end 67.23899 96.43861) (width 0.25) (layer B.Cu) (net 39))
 (segment (start 67.23899 96.43861) (end 68.4276 95.25) (width 0.25) (layer B.Cu) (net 39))
 (segment (start 68.4276 95.25) (end 68.58 95.25) (width 0.25) (layer B.Cu) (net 39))
 (segment (start 68.7324 95.25) (end 68.58 95.25) (width 0.25) (layer B.Cu) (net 39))
 (segment (start 76.38 144.5) (end 76.38 139.24359) (width 0.25) (layer B.Cu) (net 40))
 (segment (start 76.38 139.24359) (end 68.58 131.44359) (width 0.25) (layer B.Cu) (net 40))
 (segment (start 68.58 131.44359) (end 68.58 103.9836) (width 0.25) (layer B.Cu) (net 40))
 (segment (start 68.58 103.9836) (end 68.58 102.87) (width 0.25) (layer B.Cu) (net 40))
 (segment (start 68.58 69.85) (end 65.53 69.85) (width 0.25) (layer B.Cu) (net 2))
 (segment (start 65.53 69.85) (end 63.5 71.88) (width 0.25) (layer B.Cu) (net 2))
 (segment (start 61.77 122.5) (end 61.77 106.746398) (width 0.25) (layer B.Cu) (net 2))
 (segment (start 70.358 69.85) (end 68.58 69.85) (width 0.25) (layer B.Cu) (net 2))
 (segment (start 71.12 70.612) (end 70.358 69.85) (width 0.25) (layer B.Cu) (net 2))
 (segment (start 71.12 73.152) (end 71.12 70.612) (width 0.25) (layer B.Cu) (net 2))
 (segment (start 70.612 73.66) (end 71.12 73.152) (width 0.25) (layer B.Cu) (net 2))
 (segment (start 66.04 73.66) (end 70.612 73.66) (width 0.25) (layer B.Cu) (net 2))
 (segment (start 65.274493 74.425507) (end 66.04 73.66) (width 0.25) (layer B.Cu) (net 2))
 (segment (start 65.274493 103.241905) (end 65.274493 74.425507) (width 0.25) (layer B.Cu) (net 2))
 (segment (start 61.77 106.746398) (end 65.274493 103.241905) (width 0.25) (layer B.Cu) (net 2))
 (segment (start 78.42 111) (end 78.42 109.734) (width 0.25) (layer B.Cu) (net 2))
 (segment (start 78.42 109.734) (end 78.34499 109.65899) (width 0.25) (layer B.Cu) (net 2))
 (segment (start 78.34499 109.65899) (end 75.387662 109.65899) (width 0.25) (layer B.Cu) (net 2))
 (segment (start 75.387662 109.65899) (end 74.69139 110.355262) (width 0.25) (layer B.Cu) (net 2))
 (segment (start 74.69139 110.355262) (end 74.69139 131.06769) (width 0.25) (layer B.Cu) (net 2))
 (segment (start 74.69139 131.06769) (end 80.23 136.6063) (width 0.25) (layer B.Cu) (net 2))
 (segment (start 80.23 136.6063) (end 80.23 137) (width 0.25) (layer B.Cu) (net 2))
 (segment (start 78.42 111) (end 78.42 111.1524) (width 0.25) (layer B.Cu) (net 2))
 (segment (start 85.852 141.585766) (end 85.344 141.585766) (width 0.25) (layer B.Cu) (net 2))
 (segment (start 85.344 141.585766) (end 81.133766 141.585766) (width 0.25) (layer B.Cu) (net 2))
 (segment (start 61.77 122.8937) (end 58.175509 126.488191) (width 0.25) (layer B.Cu) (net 2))
 (segment (start 85.344 145.116248) (end 85.344 141.585766) (width 0.25) (layer B.Cu) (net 2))
 (segment (start 61.77 122.5) (end 61.77 122.8937) (width 0.25) (layer B.Cu) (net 2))
 (segment (start 58.175509 126.488191) (end 58.175509 138.255757) (width 0.25) (layer B.Cu) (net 2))
 (segment (start 74.479991 145.196649) (end 75.783352 146.50001) (width 0.25) (layer B.Cu) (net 2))
 (segment (start 58.175509 138.255757) (end 58.864243 138.944491) (width 0.25) (layer B.Cu) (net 2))
 (segment (start 75.783352 146.50001) (end 83.960238 146.50001) (width 0.25) (layer B.Cu) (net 2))
 (segment (start 58.864243 138.944491) (end 73.920491 138.944491) (width 0.25) (layer B.Cu) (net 2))
 (segment (start 73.920491 138.944491) (end 74.47999 139.50399) (width 0.25) (layer B.Cu) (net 2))
 (segment (start 74.47999 139.50399) (end 74.479991 145.196649) (width 0.25) (layer B.Cu) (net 2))
 (segment (start 83.960238 146.50001) (end 85.344 145.116248) (width 0.25) (layer B.Cu) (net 2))
 (segment (start 94.8455 141.585766) (end 85.852 141.585766) (width 0.25) (layer B.Cu) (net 2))
 (segment (start 81.133766 141.585766) (end 80.23 140.682) (width 0.25) (layer B.Cu) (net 2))
 (segment (start 80.23 140.682) (end 80.23 137) (width 0.25) (layer B.Cu) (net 2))
 (segment (start 98.675509 137.755757) (end 94.8455 141.585766) (width 0.25) (layer B.Cu) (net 2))
 (segment (start 97.73 122.8937) (end 101.65799 126.82169) (width 0.25) (layer B.Cu) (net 2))
 (segment (start 101.65799 133.501762) (end 98.675509 136.484243) (width 0.25) (layer B.Cu) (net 2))
 (segment (start 98.675509 136.484243) (end 98.675509 137.755757) (width 0.25) (layer B.Cu) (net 2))
 (segment (start 101.65799 126.82169) (end 101.65799 133.501762) (width 0.25) (layer B.Cu) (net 2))
 (segment (start 80.23 137.3937) (end 80.23 137) (width 0.25) (layer B.Cu) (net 2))
 (segment (start 97.73 122.5) (end 97.73 122.8937) (width 0.25) (layer B.Cu) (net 2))
 (segment (start 96.5 71.88) (end 92.9 71.88) (width 0.25) (layer B.Cu) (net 19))
 (segment (start 92.9 71.88) (end 92.266 71.246) (width 0.25) (layer B.Cu) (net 19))
 (segment (start 92.266 71.246) (end 92.266 71.0936) (width 0.25) (layer B.Cu) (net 19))
 (segment (start 92.266 71.0936) (end 91.1524 69.98) (width 0.25) (layer B.Cu) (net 19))
 (segment (start 91.1524 69.98) (end 91 69.98) (width 0.25) (layer B.Cu) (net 19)))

